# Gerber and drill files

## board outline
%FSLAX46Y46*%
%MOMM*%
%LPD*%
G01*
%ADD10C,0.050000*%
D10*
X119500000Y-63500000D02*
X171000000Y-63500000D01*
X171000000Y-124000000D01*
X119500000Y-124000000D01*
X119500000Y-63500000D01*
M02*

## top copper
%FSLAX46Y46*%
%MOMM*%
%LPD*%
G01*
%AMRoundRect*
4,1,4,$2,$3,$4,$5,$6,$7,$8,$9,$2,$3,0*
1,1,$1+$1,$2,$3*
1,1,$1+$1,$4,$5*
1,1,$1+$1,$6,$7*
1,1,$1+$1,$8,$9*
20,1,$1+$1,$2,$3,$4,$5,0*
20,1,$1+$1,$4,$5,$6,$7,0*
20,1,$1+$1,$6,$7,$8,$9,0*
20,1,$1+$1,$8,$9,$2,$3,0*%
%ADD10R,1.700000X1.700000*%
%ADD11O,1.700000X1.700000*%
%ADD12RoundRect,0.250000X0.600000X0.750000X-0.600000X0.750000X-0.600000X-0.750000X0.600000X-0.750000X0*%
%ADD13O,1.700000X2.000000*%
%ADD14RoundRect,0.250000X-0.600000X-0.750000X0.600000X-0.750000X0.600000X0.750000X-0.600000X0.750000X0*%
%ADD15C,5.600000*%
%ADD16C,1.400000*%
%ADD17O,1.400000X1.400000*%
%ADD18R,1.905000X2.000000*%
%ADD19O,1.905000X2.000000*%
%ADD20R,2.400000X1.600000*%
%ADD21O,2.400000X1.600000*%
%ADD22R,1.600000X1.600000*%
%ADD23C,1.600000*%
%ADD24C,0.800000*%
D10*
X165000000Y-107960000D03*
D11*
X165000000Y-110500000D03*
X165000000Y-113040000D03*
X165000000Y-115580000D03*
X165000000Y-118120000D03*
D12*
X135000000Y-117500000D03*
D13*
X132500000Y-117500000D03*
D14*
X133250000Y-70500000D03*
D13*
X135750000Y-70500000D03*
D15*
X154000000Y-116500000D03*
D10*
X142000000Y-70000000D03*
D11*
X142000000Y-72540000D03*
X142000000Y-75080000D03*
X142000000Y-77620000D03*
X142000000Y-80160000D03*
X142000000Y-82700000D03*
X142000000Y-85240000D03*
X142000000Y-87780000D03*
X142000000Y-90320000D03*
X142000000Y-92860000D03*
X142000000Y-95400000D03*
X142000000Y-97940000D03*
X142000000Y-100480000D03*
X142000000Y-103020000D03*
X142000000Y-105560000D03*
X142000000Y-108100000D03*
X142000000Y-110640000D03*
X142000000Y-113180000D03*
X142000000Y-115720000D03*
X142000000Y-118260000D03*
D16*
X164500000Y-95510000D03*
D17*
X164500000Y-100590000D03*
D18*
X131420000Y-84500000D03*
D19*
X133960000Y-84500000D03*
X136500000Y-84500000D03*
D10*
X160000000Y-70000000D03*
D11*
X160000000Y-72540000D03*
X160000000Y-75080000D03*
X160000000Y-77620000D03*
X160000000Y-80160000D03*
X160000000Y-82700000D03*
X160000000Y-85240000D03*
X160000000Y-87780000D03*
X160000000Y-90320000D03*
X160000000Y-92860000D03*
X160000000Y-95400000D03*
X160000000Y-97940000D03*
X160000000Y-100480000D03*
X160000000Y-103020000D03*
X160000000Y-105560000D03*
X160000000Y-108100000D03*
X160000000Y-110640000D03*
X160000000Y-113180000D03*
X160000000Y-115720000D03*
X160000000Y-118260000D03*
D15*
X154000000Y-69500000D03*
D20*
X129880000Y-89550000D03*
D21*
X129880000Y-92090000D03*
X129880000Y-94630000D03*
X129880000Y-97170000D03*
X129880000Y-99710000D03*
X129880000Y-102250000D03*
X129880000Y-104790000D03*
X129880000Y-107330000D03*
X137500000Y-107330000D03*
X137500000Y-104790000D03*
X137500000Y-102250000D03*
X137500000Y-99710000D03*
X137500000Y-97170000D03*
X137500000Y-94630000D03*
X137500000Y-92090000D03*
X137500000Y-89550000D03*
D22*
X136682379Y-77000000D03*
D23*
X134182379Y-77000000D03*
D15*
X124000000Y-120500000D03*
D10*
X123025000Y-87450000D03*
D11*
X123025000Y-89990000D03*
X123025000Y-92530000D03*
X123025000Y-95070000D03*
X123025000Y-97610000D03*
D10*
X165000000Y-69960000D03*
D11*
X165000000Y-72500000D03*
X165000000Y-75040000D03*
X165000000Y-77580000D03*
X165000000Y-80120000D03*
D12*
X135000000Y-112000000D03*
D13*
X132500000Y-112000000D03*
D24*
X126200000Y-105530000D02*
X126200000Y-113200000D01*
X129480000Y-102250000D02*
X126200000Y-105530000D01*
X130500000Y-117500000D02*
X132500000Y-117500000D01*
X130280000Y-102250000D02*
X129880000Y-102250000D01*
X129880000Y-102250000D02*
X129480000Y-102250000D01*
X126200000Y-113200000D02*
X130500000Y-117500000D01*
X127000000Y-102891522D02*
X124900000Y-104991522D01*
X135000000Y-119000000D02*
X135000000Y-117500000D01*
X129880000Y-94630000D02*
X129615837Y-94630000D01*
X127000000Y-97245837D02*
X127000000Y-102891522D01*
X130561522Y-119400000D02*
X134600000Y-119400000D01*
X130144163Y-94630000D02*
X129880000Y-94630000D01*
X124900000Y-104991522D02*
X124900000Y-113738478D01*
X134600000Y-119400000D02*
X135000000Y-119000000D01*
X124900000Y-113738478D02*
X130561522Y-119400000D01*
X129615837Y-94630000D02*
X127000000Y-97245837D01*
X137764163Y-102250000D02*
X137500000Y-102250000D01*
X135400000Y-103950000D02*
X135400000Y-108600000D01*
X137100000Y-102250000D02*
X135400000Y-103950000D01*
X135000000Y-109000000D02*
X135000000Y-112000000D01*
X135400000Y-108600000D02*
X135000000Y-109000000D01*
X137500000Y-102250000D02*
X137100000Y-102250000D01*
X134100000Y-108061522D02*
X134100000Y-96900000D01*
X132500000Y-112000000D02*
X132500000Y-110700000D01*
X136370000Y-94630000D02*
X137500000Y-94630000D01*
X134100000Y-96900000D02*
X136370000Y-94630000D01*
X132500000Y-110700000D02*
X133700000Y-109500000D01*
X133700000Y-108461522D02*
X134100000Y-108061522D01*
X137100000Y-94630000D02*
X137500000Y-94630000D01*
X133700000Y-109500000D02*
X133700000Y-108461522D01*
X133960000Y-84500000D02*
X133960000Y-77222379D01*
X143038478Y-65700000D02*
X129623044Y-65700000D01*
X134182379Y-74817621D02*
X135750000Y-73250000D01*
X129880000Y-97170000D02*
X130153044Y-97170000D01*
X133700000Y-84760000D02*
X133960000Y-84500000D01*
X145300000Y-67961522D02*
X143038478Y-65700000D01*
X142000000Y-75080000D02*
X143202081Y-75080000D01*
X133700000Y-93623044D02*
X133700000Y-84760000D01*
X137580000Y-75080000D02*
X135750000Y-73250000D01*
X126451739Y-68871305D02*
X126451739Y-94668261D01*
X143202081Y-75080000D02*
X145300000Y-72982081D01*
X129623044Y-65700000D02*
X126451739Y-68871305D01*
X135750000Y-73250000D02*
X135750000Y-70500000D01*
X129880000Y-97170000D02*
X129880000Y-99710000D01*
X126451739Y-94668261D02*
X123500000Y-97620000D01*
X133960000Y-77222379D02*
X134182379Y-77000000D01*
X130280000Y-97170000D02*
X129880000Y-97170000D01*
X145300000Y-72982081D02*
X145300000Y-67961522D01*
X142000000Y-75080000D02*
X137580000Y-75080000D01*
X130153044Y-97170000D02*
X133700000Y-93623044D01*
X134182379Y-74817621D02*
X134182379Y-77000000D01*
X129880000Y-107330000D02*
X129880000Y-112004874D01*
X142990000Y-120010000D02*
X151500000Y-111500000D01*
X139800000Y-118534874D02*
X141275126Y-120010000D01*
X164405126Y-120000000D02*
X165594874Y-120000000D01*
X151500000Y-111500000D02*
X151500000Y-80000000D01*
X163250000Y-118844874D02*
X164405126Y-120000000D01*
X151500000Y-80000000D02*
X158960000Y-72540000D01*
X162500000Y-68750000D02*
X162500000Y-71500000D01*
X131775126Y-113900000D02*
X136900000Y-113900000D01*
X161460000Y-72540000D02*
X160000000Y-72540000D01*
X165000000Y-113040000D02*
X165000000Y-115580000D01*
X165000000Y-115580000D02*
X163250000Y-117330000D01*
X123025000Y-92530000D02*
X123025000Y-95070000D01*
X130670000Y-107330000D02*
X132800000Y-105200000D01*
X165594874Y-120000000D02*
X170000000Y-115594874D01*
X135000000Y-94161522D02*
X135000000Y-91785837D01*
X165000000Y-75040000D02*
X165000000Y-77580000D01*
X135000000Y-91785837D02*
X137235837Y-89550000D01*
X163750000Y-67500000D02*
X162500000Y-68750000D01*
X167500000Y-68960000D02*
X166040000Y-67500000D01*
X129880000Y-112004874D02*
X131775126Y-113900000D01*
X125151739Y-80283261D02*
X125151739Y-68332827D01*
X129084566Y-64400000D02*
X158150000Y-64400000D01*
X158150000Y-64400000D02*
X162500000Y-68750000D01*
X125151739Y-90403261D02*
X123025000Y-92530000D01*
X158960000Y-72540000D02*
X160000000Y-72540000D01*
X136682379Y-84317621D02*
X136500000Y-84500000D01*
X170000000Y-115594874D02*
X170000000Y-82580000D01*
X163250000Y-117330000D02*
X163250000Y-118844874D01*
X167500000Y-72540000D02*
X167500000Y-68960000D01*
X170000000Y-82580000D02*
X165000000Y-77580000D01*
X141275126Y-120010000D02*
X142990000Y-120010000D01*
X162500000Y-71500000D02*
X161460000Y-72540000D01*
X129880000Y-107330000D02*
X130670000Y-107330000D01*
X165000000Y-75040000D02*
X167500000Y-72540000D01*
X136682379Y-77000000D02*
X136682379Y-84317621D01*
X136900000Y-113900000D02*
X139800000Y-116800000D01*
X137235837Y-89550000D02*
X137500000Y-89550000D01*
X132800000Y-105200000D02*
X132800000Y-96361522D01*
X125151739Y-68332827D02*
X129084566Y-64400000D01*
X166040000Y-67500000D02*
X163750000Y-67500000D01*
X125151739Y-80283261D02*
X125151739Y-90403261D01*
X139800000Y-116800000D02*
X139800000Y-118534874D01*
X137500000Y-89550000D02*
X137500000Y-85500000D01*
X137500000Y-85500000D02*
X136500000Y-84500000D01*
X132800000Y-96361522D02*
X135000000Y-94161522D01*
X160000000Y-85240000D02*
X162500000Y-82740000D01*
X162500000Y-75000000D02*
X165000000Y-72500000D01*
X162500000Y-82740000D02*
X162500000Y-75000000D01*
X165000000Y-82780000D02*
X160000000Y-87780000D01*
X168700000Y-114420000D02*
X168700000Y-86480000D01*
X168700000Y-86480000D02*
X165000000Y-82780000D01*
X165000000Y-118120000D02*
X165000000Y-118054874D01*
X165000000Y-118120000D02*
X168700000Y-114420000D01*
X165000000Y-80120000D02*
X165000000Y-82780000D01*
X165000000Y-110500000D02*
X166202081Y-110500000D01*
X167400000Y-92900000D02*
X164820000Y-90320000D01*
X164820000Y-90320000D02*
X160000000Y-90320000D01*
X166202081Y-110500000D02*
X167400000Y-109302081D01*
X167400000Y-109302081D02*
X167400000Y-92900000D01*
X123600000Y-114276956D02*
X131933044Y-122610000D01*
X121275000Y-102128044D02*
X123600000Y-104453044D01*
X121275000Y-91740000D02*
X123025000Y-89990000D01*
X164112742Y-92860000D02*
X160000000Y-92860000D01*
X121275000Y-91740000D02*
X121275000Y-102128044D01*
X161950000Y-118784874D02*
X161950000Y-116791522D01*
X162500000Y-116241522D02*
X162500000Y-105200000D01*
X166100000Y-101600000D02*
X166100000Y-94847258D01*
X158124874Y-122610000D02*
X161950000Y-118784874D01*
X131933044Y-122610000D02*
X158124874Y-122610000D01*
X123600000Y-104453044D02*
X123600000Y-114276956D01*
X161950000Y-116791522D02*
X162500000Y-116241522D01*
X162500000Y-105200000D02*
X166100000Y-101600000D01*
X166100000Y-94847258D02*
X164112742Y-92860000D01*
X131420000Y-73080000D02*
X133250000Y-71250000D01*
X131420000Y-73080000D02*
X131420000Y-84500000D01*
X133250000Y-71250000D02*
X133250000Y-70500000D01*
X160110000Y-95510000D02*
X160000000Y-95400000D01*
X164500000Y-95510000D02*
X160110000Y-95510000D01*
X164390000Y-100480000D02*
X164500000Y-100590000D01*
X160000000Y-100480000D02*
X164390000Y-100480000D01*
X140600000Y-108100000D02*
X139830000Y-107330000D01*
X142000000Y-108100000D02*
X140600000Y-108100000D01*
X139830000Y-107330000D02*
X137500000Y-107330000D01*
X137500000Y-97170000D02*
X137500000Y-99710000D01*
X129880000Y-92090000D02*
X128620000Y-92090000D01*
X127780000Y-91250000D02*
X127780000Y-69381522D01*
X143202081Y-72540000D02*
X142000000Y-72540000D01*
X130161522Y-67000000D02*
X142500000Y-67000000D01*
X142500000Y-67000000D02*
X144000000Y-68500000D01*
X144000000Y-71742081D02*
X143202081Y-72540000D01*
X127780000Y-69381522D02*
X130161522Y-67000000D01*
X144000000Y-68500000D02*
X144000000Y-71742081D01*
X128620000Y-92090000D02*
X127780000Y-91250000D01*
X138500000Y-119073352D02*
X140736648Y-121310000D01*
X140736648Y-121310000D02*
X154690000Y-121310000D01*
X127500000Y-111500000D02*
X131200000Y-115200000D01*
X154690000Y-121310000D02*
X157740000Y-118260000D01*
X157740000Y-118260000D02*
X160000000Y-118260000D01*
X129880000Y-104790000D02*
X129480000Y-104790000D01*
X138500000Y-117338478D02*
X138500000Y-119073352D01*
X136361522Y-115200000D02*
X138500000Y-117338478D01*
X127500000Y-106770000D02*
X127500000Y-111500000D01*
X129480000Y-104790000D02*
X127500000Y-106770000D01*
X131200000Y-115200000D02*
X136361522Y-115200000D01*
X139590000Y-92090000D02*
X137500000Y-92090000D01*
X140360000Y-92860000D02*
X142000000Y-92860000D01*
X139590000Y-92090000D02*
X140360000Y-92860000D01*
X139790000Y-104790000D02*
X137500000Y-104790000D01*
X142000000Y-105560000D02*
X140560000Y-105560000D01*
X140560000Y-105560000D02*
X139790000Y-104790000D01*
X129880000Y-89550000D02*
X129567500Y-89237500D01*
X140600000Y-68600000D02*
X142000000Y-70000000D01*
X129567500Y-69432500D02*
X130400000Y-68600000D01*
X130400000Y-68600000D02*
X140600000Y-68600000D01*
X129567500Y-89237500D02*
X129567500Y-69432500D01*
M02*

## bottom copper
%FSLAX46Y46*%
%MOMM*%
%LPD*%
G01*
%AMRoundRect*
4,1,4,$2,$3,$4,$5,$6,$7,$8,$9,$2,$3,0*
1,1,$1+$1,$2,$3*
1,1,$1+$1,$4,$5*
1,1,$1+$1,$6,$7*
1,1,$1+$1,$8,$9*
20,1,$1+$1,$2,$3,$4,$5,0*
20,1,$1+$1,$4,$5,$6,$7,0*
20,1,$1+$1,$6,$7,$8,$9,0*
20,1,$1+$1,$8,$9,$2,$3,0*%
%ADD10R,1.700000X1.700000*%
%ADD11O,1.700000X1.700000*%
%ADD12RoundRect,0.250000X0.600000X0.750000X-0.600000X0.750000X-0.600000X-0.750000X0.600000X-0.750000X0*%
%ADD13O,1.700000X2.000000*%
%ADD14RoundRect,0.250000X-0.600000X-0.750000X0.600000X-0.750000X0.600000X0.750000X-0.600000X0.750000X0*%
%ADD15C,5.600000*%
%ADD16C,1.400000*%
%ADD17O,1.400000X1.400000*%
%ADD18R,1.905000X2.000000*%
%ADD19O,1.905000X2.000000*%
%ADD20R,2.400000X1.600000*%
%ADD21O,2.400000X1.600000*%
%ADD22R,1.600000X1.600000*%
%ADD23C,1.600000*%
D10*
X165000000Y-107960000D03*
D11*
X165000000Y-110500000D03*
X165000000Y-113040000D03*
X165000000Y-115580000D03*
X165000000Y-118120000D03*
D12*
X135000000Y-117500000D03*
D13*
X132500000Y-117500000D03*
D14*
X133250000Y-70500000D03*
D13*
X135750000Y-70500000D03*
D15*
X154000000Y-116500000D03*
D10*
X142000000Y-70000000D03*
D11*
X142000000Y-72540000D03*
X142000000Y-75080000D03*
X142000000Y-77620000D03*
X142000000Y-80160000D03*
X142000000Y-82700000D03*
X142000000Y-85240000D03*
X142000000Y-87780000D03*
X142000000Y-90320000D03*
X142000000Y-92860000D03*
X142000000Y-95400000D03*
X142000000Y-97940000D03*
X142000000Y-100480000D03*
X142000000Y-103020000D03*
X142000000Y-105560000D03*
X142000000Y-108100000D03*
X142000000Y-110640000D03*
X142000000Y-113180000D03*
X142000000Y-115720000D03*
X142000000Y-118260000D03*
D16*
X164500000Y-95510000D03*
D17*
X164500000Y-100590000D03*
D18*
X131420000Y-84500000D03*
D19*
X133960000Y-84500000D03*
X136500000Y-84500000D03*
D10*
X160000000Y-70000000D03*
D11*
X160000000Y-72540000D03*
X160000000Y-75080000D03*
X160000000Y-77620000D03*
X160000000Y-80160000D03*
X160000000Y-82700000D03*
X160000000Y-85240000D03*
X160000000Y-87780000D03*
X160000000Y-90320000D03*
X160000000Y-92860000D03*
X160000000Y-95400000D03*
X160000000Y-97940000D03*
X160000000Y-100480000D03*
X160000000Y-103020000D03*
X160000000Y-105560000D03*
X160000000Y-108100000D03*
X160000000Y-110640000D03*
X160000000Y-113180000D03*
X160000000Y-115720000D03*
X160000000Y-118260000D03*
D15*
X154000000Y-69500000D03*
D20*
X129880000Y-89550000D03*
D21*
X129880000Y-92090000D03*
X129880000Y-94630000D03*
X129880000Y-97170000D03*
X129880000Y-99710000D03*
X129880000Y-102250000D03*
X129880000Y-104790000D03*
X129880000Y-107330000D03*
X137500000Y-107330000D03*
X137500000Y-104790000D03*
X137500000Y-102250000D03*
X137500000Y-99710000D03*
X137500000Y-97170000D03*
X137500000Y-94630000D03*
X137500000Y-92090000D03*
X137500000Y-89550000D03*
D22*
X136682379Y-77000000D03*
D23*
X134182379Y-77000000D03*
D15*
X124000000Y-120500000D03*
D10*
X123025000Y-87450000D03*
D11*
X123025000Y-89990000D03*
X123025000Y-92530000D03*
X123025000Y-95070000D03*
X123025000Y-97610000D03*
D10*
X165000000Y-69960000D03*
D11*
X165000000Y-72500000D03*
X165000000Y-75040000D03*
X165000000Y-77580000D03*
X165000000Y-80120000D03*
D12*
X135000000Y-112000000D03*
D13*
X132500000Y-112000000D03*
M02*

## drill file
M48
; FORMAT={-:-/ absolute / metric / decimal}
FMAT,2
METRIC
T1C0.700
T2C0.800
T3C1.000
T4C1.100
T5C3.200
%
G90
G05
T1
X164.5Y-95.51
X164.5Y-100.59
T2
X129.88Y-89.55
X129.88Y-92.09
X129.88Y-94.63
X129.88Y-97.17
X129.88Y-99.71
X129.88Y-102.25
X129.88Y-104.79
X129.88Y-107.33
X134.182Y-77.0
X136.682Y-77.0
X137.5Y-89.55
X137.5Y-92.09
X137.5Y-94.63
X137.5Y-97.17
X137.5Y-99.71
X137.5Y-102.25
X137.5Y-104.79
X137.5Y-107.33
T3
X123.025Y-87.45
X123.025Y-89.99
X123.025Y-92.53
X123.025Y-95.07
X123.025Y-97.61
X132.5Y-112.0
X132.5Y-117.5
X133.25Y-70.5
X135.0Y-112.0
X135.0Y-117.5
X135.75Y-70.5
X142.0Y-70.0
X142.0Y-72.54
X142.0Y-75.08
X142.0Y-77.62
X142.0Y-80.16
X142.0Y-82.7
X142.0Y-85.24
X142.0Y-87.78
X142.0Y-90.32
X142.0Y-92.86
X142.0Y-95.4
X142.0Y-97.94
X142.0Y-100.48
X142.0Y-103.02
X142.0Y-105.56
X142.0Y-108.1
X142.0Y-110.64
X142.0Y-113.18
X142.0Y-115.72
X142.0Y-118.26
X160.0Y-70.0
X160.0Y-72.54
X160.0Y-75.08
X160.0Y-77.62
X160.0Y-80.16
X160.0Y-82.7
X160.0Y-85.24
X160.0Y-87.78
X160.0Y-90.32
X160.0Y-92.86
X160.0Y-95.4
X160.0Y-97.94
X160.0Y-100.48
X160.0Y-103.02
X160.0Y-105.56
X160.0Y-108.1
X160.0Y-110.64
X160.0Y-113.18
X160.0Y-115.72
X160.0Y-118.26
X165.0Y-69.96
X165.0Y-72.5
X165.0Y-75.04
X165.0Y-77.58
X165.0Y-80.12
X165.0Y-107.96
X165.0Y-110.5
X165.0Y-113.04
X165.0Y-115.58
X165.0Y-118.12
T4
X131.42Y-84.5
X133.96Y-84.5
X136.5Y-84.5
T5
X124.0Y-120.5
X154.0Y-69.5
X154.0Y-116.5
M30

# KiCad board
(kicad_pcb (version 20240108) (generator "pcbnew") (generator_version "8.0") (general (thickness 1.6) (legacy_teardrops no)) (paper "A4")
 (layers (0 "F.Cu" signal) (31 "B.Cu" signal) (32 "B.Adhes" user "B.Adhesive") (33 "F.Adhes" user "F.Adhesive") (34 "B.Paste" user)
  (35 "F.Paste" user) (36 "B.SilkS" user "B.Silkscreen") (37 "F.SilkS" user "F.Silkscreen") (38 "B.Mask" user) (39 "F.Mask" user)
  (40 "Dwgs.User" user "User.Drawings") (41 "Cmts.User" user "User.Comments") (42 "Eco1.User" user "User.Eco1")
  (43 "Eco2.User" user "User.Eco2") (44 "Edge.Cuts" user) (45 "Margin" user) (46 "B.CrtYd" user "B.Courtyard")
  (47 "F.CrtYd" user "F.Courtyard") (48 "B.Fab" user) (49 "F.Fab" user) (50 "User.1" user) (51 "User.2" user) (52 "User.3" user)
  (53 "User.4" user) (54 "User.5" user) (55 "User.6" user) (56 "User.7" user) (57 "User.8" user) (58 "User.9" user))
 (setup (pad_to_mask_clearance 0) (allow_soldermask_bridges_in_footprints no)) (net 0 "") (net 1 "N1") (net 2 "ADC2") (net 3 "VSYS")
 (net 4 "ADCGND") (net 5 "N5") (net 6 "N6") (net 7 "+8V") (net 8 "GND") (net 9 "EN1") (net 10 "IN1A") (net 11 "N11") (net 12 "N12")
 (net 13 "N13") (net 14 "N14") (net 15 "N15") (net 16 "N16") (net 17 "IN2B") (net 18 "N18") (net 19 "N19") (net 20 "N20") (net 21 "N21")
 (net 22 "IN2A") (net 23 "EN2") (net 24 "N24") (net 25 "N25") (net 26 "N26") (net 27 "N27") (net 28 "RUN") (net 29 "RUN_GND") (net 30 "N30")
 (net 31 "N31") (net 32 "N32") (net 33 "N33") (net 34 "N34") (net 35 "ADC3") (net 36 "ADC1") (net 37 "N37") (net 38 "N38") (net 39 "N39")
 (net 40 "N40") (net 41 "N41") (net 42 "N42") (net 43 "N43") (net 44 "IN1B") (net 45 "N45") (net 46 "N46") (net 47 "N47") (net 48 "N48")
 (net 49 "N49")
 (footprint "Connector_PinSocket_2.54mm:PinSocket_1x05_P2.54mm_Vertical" (layer "F.Cu") (at 165 107.96)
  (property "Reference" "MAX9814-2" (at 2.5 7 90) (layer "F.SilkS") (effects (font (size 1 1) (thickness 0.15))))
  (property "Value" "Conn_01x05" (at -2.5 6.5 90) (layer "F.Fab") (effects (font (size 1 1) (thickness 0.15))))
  (pad "1" thru_hole rect (at 0 0) (size 1.7 1.7) (drill 1) (layers "*.Cu" "*.Mask") (remove_unused_layers no) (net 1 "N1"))
  (pad "2" thru_hole oval (at 0 2.54) (size 1.7 1.7) (drill 1) (layers "*.Cu" "*.Mask") (remove_unused_layers no) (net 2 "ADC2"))
  (pad "3" thru_hole oval (at 0 5.08) (size 1.7 1.7) (drill 1) (layers "*.Cu" "*.Mask") (remove_unused_layers no) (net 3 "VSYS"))
  (pad "4" thru_hole oval (at 0 7.62) (size 1.7 1.7) (drill 1) (layers "*.Cu" "*.Mask") (remove_unused_layers no) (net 3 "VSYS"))
  (pad "5" thru_hole oval (at 0 10.16) (size 1.7 1.7) (drill 1) (layers "*.Cu" "*.Mask") (remove_unused_layers no) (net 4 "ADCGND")))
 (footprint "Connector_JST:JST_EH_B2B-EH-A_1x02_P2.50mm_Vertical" (layer "F.Cu") (at 135 117.5 180)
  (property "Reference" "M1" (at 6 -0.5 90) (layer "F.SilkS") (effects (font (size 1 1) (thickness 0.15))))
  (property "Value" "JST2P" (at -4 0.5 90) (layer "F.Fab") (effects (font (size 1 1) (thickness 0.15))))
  (pad "1" thru_hole roundrect (at 0 0 180) (size 1.7 2) (drill 1) (layers "*.Cu" "*.Mask") (remove_unused_layers no)
   (roundrect_rratio 0.147059) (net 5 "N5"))
  (pad "2" thru_hole oval (at 2.5 0 180) (size 1.7 2) (drill 1) (layers "*.Cu" "*.Mask") (remove_unused_layers no) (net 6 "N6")))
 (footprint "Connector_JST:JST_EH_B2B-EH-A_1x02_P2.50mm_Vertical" (layer "F.Cu") (at 133.25 70.5)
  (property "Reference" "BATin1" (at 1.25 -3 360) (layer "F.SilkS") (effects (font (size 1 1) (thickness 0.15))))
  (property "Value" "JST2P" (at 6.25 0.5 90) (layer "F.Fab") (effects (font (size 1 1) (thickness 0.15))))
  (pad "1" thru_hole roundrect (at 0 0) (size 1.7 2) (drill 1) (layers "*.Cu" "*.Mask") (remove_unused_layers no)
   (roundrect_rratio 0.147059) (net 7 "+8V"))
  (pad "2" thru_hole oval (at 2.5 0) (size 1.7 2) (drill 1) (layers "*.Cu" "*.Mask") (remove_unused_layers no) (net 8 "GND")))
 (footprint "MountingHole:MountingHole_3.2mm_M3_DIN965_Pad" (layer "F.Cu") (at 154 116.5)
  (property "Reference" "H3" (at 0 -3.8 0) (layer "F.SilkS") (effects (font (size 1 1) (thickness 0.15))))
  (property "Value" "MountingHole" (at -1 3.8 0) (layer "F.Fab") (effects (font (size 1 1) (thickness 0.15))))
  (pad "1" thru_hole circle (at 0 0) (size 5.6 5.6) (drill 3.2) (layers "*.Cu" "*.Mask") (remove_unused_layers no)))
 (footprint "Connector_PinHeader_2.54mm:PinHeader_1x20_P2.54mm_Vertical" (layer "F.Cu") (at 142 70)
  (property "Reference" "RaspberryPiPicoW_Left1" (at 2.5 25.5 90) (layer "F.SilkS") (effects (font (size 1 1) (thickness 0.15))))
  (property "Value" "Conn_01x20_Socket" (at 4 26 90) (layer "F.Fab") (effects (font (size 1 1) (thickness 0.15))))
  (pad "1" thru_hole rect (at 0 0) (size 1.7 1.7) (drill 1) (layers "*.Cu" "*.Mask") (remove_unused_layers no) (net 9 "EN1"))
  (pad "2" thru_hole oval (at 0 2.54) (size 1.7 1.7) (drill 1) (layers "*.Cu" "*.Mask") (remove_unused_layers no) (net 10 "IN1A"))
  (pad "3" thru_hole oval (at 0 5.08) (size 1.7 1.7) (drill 1) (layers "*.Cu" "*.Mask") (remove_unused_layers no) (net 8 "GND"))
  (pad "4" thru_hole oval (at 0 7.62) (size 1.7 1.7) (drill 1) (layers "*.Cu" "*.Mask") (remove_unused_layers no) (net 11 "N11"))
  (pad "5" thru_hole oval (at 0 10.16) (size 1.7 1.7) (drill 1) (layers "*.Cu" "*.Mask") (remove_unused_layers no) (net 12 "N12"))
  (pad "6" thru_hole oval (at 0 12.7) (size 1.7 1.7) (drill 1) (layers "*.Cu" "*.Mask") (remove_unused_layers no) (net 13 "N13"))
  (pad "7" thru_hole oval (at 0 15.24) (size 1.7 1.7) (drill 1) (layers "*.Cu" "*.Mask") (remove_unused_layers no) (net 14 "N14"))
  (pad "8" thru_hole oval (at 0 17.78) (size 1.7 1.7) (drill 1) (layers "*.Cu" "*.Mask") (remove_unused_layers no) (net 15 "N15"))
  (pad "9" thru_hole oval (at 0 20.32) (size 1.7 1.7) (drill 1) (layers "*.Cu" "*.Mask") (remove_unused_layers no) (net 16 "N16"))
  (pad "10" thru_hole oval (at 0 22.86) (size 1.7 1.7) (drill 1) (layers "*.Cu" "*.Mask") (remove_unused_layers no) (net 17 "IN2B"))
  (pad "11" thru_hole oval (at 0 25.4) (size 1.7 1.7) (drill 1) (layers "*.Cu" "*.Mask") (remove_unused_layers no) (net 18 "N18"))
  (pad "12" thru_hole oval (at 0 27.94) (size 1.7 1.7) (drill 1) (layers "*.Cu" "*.Mask") (remove_unused_layers no) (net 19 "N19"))
  (pad "13" thru_hole oval (at 0 30.48) (size 1.7 1.7) (drill 1) (layers "*.Cu" "*.Mask") (remove_unused_layers no) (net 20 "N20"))
  (pad "14" thru_hole oval (at 0 33.02) (size 1.7 1.7) (drill 1) (layers "*.Cu" "*.Mask") (remove_unused_layers no) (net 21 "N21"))
  (pad "15" thru_hole oval (at 0 35.56) (size 1.7 1.7) (drill 1) (layers "*.Cu" "*.Mask") (remove_unused_layers no) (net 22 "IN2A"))
  (pad "16" thru_hole oval (at 0 38.1) (size 1.7 1.7) (drill 1) (layers "*.Cu" "*.Mask") (remove_unused_layers no) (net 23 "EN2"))
  (pad "17" thru_hole oval (at 0 40.64) (size 1.7 1.7) (drill 1) (layers "*.Cu" "*.Mask") (remove_unused_layers no) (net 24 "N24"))
  (pad "18" thru_hole oval (at 0 43.18) (size 1.7 1.7) (drill 1) (layers "*.Cu" "*.Mask") (remove_unused_layers no) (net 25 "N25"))
  (pad "19" thru_hole oval (at 0 45.72) (size 1.7 1.7) (drill 1) (layers "*.Cu" "*.Mask") (remove_unused_layers no) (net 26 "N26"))
  (pad "20" thru_hole oval (at 0 48.26) (size 1.7 1.7) (drill 1) (layers "*.Cu" "*.Mask") (remove_unused_layers no) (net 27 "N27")))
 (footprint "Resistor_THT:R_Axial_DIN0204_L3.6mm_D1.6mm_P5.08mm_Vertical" (layer "F.Cu") (at 164.5 95.51 -90)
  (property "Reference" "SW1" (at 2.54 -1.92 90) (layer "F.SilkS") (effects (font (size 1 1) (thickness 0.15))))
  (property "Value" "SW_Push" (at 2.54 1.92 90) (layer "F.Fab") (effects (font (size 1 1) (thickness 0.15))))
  (pad "1" thru_hole circle (at 0 0 270) (size 1.4 1.4) (drill 0.7) (layers "*.Cu" "*.Mask") (remove_unused_layers no) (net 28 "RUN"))
  (pad "2" thru_hole oval (at 5.08 0 270) (size 1.4 1.4) (drill 0.7) (layers "*.Cu" "*.Mask") (remove_unused_layers no) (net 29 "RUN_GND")))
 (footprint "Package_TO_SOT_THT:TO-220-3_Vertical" (layer "F.Cu") (at 131.42 84.5)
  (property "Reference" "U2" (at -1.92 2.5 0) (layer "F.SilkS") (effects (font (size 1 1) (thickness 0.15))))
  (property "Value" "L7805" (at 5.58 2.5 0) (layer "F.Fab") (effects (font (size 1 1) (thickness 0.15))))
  (pad "1" thru_hole rect (at 0 0) (size 1.905 2) (drill 1.1) (layers "*.Cu" "*.Mask") (remove_unused_layers no) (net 7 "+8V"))
  (pad "2" thru_hole oval (at 2.54 0) (size 1.905 2) (drill 1.1) (layers "*.Cu" "*.Mask") (remove_unused_layers no) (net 8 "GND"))
  (pad "3" thru_hole oval (at 5.08 0) (size 1.905 2) (drill 1.1) (layers "*.Cu" "*.Mask") (remove_unused_layers no) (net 3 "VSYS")))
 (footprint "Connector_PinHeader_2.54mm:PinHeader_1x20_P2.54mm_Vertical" (layer "F.Cu") (at 160 70)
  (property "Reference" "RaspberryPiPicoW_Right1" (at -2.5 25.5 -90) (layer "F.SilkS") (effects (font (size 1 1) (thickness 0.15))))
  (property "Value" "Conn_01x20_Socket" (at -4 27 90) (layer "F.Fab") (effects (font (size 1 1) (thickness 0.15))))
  (pad "1" thru_hole rect (at 0 0) (size 1.7 1.7) (drill 1) (layers "*.Cu" "*.Mask") (remove_unused_layers no) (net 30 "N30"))
  (pad "2" thru_hole oval (at 0 2.54) (size 1.7 1.7) (drill 1) (layers "*.Cu" "*.Mask") (remove_unused_layers no) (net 3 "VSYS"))
  (pad "3" thru_hole oval (at 0 5.08) (size 1.7 1.7) (drill 1) (layers "*.Cu" "*.Mask") (remove_unused_layers no) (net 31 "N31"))
  (pad "4" thru_hole oval (at 0 7.62) (size 1.7 1.7) (drill 1) (layers "*.Cu" "*.Mask") (remove_unused_layers no) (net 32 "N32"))
  (pad "5" thru_hole oval (at 0 10.16) (size 1.7 1.7) (drill 1) (layers "*.Cu" "*.Mask") (remove_unused_layers no) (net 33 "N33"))
  (pad "6" thru_hole oval (at 0 12.7) (size 1.7 1.7) (drill 1) (layers "*.Cu" "*.Mask") (remove_unused_layers no) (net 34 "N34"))
  (pad "7" thru_hole oval (at 0 15.24) (size 1.7 1.7) (drill 1) (layers "*.Cu" "*.Mask") (remove_unused_layers no) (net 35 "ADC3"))
  (pad "8" thru_hole oval (at 0 17.78) (size 1.7 1.7) (drill 1) (layers "*.Cu" "*.Mask") (remove_unused_layers no) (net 4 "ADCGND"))
  (pad "9" thru_hole oval (at 0 20.32) (size 1.7 1.7) (drill 1) (layers "*.Cu" "*.Mask") (remove_unused_layers no) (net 2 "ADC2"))
  (pad "10" thru_hole oval (at 0 22.86) (size 1.7 1.7) (drill 1) (layers "*.Cu" "*.Mask") (remove_unused_layers no) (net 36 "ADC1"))
  (pad "11" thru_hole oval (at 0 25.4) (size 1.7 1.7) (drill 1) (layers "*.Cu" "*.Mask") (remove_unused_layers no) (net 28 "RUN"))
  (pad "12" thru_hole oval (at 0 27.94) (size 1.7 1.7) (drill 1) (layers "*.Cu" "*.Mask") (remove_unused_layers no) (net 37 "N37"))
  (pad "13" thru_hole oval (at 0 30.48) (size 1.7 1.7) (drill 1) (layers "*.Cu" "*.Mask") (remove_unused_layers no) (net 29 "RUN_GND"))
  (pad "14" thru_hole oval (at 0 33.02) (size 1.7 1.7) (drill 1) (layers "*.Cu" "*.Mask") (remove_unused_layers no) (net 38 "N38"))
  (pad "15" thru_hole oval (at 0 35.56) (size 1.7 1.7) (drill 1) (layers "*.Cu" "*.Mask") (remove_unused_layers no) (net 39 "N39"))
  (pad "16" thru_hole oval (at 0 38.1) (size 1.7 1.7) (drill 1) (layers "*.Cu" "*.Mask") (remove_unused_layers no) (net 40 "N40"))
  (pad "17" thru_hole oval (at 0 40.64) (size 1.7 1.7) (drill 1) (layers "*.Cu" "*.Mask") (remove_unused_layers no) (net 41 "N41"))
  (pad "18" thru_hole oval (at 0 43.18) (size 1.7 1.7) (drill 1) (layers "*.Cu" "*.Mask") (remove_unused_layers no) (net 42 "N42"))
  (pad "19" thru_hole oval (at 0 45.72) (size 1.7 1.7) (drill 1) (layers "*.Cu" "*.Mask") (remove_unused_layers no) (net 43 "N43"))
  (pad "20" thru_hole oval (at 0 48.26) (size 1.7 1.7) (drill 1) (layers "*.Cu" "*.Mask") (remove_unused_layers no) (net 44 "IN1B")))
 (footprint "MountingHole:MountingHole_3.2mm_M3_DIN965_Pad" (layer "F.Cu") (at 154 69.5)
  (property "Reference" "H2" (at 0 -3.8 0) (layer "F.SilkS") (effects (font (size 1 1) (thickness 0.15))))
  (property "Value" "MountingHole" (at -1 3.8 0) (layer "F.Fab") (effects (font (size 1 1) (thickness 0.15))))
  (pad "1" thru_hole circle (at 0 0) (size 5.6 5.6) (drill 3.2) (layers "*.Cu" "*.Mask") (remove_unused_layers no)))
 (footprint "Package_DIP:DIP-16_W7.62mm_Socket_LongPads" (layer "F.Cu") (at 129.88 89.55)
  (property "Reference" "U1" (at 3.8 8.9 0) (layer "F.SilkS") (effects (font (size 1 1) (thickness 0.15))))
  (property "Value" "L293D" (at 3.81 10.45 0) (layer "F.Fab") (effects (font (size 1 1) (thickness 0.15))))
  (pad "1" thru_hole rect (at 0 0) (size 2.4 1.6) (drill 0.8) (layers "*.Cu" "*.Mask") (remove_unused_layers no) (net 9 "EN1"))
  (pad "2" thru_hole oval (at 0 2.54) (size 2.4 1.6) (drill 0.8) (layers "*.Cu" "*.Mask") (remove_unused_layers no) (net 10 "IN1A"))
  (pad "3" thru_hole oval (at 0 5.08) (size 2.4 1.6) (drill 0.8) (layers "*.Cu" "*.Mask") (remove_unused_layers no) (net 5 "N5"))
  (pad "4" thru_hole oval (at 0 7.62) (size 2.4 1.6) (drill 0.8) (layers "*.Cu" "*.Mask") (remove_unused_layers no) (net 8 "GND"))
  (pad "5" thru_hole oval (at 0 10.16) (size 2.4 1.6) (drill 0.8) (layers "*.Cu" "*.Mask") (remove_unused_layers no) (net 8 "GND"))
  (pad "6" thru_hole oval (at 0 12.7) (size 2.4 1.6) (drill 0.8) (layers "*.Cu" "*.Mask") (remove_unused_layers no) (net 6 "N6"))
  (pad "7" thru_hole oval (at 0 15.24) (size 2.4 1.6) (drill 0.8) (layers "*.Cu" "*.Mask") (remove_unused_layers no) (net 44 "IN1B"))
  (pad "8" thru_hole oval (at 0 17.78) (size 2.4 1.6) (drill 0.8) (layers "*.Cu" "*.Mask") (remove_unused_layers no) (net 3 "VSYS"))
  (pad "9" thru_hole oval (at 7.62 17.78) (size 2.4 1.6) (drill 0.8) (layers "*.Cu" "*.Mask") (remove_unused_layers no) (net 23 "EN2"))
  (pad "10" thru_hole oval (at 7.62 15.24) (size 2.4 1.6) (drill 0.8) (layers "*.Cu" "*.Mask") (remove_unused_layers no) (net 22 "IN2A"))
  (pad "11" thru_hole oval (at 7.62 12.7) (size 2.4 1.6) (drill 0.8) (layers "*.Cu" "*.Mask") (remove_unused_layers no) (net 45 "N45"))
  (pad "12" thru_hole oval (at 7.62 10.16) (size 2.4 1.6) (drill 0.8) (layers "*.Cu" "*.Mask") (remove_unused_layers no) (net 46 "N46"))
  (pad "13" thru_hole oval (at 7.62 7.62) (size 2.4 1.6) (drill 0.8) (layers "*.Cu" "*.Mask") (remove_unused_layers no) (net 46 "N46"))
  (pad "14" thru_hole oval (at 7.62 5.08) (size 2.4 1.6) (drill 0.8) (layers "*.Cu" "*.Mask") (remove_unused_layers no) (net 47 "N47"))
  (pad "15" thru_hole oval (at 7.62 2.54) (size 2.4 1.6) (drill 0.8) (layers "*.Cu" "*.Mask") (remove_unused_layers no) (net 17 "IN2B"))
  (pad "16" thru_hole oval (at 7.62 0) (size 2.4 1.6) (drill 0.8) (layers "*.Cu" "*.Mask") (remove_unused_layers no) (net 3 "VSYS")))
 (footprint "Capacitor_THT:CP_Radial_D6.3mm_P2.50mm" (layer "F.Cu") (at 136.682379 77 180)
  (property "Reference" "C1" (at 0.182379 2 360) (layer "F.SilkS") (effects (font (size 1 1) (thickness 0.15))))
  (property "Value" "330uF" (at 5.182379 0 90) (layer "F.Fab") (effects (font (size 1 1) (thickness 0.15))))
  (pad "1" thru_hole rect (at 0 0 180) (size 1.6 1.6) (drill 0.8) (layers "*.Cu" "*.Mask") (remove_unused_layers no) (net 3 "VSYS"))
  (pad "2" thru_hole circle (at 2.5 0 180) (size 1.6 1.6) (drill 0.8) (layers "*.Cu" "*.Mask") (remove_unused_layers no) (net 8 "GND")))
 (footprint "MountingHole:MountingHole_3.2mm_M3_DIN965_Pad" (layer "F.Cu") (at 124 120.5)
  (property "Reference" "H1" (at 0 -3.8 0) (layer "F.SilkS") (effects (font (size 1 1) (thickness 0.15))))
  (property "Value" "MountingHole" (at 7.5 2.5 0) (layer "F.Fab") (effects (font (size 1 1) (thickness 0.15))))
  (pad "1" thru_hole circle (at 0 0) (size 5.6 5.6) (drill 3.2) (layers "*.Cu" "*.Mask") (remove_unused_layers no)))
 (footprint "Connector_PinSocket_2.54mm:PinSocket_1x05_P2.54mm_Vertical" (layer "F.Cu") (at 123.025 87.45)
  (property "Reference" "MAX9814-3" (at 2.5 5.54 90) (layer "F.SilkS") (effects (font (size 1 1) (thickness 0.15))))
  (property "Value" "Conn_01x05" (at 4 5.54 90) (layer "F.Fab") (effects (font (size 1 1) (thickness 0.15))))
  (pad "1" thru_hole rect (at 0 0) (size 1.7 1.7) (drill 1) (layers "*.Cu" "*.Mask") (remove_unused_layers no) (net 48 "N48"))
  (pad "2" thru_hole oval (at 0 2.54) (size 1.7 1.7) (drill 1) (layers "*.Cu" "*.Mask") (remove_unused_layers no) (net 36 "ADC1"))
  (pad "3" thru_hole oval (at 0 5.08) (size 1.7 1.7) (drill 1) (layers "*.Cu" "*.Mask") (remove_unused_layers no) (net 3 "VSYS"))
  (pad "4" thru_hole oval (at 0 7.62) (size 1.7 1.7) (drill 1) (layers "*.Cu" "*.Mask") (remove_unused_layers no) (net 3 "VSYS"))
  (pad "5" thru_hole oval (at 0 10.16) (size 1.7 1.7) (drill 1) (layers "*.Cu" "*.Mask") (remove_unused_layers no) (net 8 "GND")))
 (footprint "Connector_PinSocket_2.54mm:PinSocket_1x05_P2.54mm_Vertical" (layer "F.Cu") (at 165 69.96)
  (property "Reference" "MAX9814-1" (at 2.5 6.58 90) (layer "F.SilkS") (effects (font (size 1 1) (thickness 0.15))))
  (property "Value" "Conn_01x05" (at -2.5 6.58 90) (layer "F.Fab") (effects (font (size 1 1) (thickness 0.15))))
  (pad "1" thru_hole rect (at 0 0) (size 1.7 1.7) (drill 1) (layers "*.Cu" "*.Mask") (remove_unused_layers no) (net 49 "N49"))
  (pad "2" thru_hole oval (at 0 2.54) (size 1.7 1.7) (drill 1) (layers "*.Cu" "*.Mask") (remove_unused_layers no) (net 35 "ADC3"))
  (pad "3" thru_hole oval (at 0 5.08) (size 1.7 1.7) (drill 1) (layers "*.Cu" "*.Mask") (remove_unused_layers no) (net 3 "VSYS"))
  (pad "4" thru_hole oval (at 0 7.62) (size 1.7 1.7) (drill 1) (layers "*.Cu" "*.Mask") (remove_unused_layers no) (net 3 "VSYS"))
  (pad "5" thru_hole oval (at 0 10.16) (size 1.7 1.7) (drill 1) (layers "*.Cu" "*.Mask") (remove_unused_layers no) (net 4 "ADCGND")))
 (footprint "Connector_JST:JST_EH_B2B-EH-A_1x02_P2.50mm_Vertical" (layer "F.Cu") (at 135 112 180)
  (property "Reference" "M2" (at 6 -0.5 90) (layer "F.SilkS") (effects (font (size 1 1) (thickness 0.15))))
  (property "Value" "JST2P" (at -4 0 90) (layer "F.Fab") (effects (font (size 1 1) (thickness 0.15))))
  (pad "1" thru_hole roundrect (at 0 0 180) (size 1.7 2) (drill 1) (layers "*.Cu" "*.Mask") (remove_unused_layers no)
   (roundrect_rratio 0.147059) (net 45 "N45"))
  (pad "2" thru_hole oval (at 2.5 0 180) (size 1.7 2) (drill 1) (layers "*.Cu" "*.Mask") (remove_unused_layers no) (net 47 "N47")))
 (gr_rect (start 119.5 63.5) (end 171 124) (stroke (width 0.05) (type default)) (fill none) (layer "Edge.Cuts"))
 (segment (start 126.2 105.53) (end 126.2 113.2) (width 0.8) (layer "F.Cu") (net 6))
 (segment (start 129.48 102.25) (end 126.2 105.53) (width 0.8) (layer "F.Cu") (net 6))
 (segment (start 130.5 117.5) (end 132.5 117.5) (width 0.8) (layer "F.Cu") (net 6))
 (segment (start 130.28 102.25) (end 129.88 102.25) (width 0.8) (layer "F.Cu") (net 6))
 (segment (start 129.88 102.25) (end 129.48 102.25) (width 0.8) (layer "F.Cu") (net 6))
 (segment (start 126.2 113.2) (end 130.5 117.5) (width 0.8) (layer "F.Cu") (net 6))
 (segment (start 127 102.891522) (end 124.9 104.991522) (width 0.8) (layer "F.Cu") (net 5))
 (segment (start 135 119) (end 135 117.5) (width 0.8) (layer "F.Cu") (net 5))
 (segment (start 129.88 94.63) (end 129.615837 94.63) (width 0.8) (layer "F.Cu") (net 5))
 (segment (start 127 97.245837) (end 127 102.891522) (width 0.8) (layer "F.Cu") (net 5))
 (segment (start 130.561522 119.4) (end 134.6 119.4) (width 0.8) (layer "F.Cu") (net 5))
 (segment (start 130.144163 94.63) (end 129.88 94.63) (width 0.8) (layer "F.Cu") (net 5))
 (segment (start 124.9 104.991522) (end 124.9 113.738478) (width 0.8) (layer "F.Cu") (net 5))
 (segment (start 134.6 119.4) (end 135 119) (width 0.8) (layer "F.Cu") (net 5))
 (segment (start 124.9 113.738478) (end 130.561522 119.4) (width 0.8) (layer "F.Cu") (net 5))
 (segment (start 129.615837 94.63) (end 127 97.245837) (width 0.8) (layer "F.Cu") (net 5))
 (segment (start 137.764163 102.25) (end 137.5 102.25) (width 0.8) (layer "F.Cu") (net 45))
 (segment (start 135.4 103.95) (end 135.4 108.6) (width 0.8) (layer "F.Cu") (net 45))
 (segment (start 137.1 102.25) (end 135.4 103.95) (width 0.8) (layer "F.Cu") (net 45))
 (segment (start 135 109) (end 135 112) (width 0.8) (layer "F.Cu") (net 45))
 (segment (start 135.4 108.6) (end 135 109) (width 0.8) (layer "F.Cu") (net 45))
 (segment (start 137.5 102.25) (end 137.1 102.25) (width 0.8) (layer "F.Cu") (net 45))
 (segment (start 134.1 108.061522) (end 134.1 96.9) (width 0.8) (layer "F.Cu") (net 47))
 (segment (start 132.5 112) (end 132.5 110.7) (width 0.8) (layer "F.Cu") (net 47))
 (segment (start 136.37 94.63) (end 137.5 94.63) (width 0.8) (layer "F.Cu") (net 47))
 (segment (start 134.1 96.9) (end 136.37 94.63) (width 0.8) (layer "F.Cu") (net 47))
 (segment (start 132.5 110.7) (end 133.7 109.5) (width 0.8) (layer "F.Cu") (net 47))
 (segment (start 133.7 108.461522) (end 134.1 108.061522) (width 0.8) (layer "F.Cu") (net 47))
 (segment (start 137.1 94.63) (end 137.5 94.63) (width 0.8) (layer "F.Cu") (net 47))
 (segment (start 133.7 109.5) (end 133.7 108.461522) (width 0.8) (layer "F.Cu") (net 47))
 (segment (start 133.96 84.5) (end 133.96 77.222379) (width 0.8) (layer "F.Cu") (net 8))
 (segment (start 143.038478 65.7) (end 129.623044 65.7) (width 0.8) (layer "F.Cu") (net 8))
 (segment (start 134.182379 74.817621) (end 135.75 73.25) (width 0.8) (layer "F.Cu") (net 8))
 (segment (start 129.88 97.17) (end 130.153044 97.17) (width 0.8) (layer "F.Cu") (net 8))
 (segment (start 133.7 84.76) (end 133.96 84.5) (width 0.8) (layer "F.Cu") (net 8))
 (segment (start 145.3 67.961522) (end 143.038478 65.7) (width 0.8) (layer "F.Cu") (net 8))
 (segment (start 142 75.08) (end 143.202081 75.08) (width 0.8) (layer "F.Cu") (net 8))
 (segment (start 133.7 93.623044) (end 133.7 84.76) (width 0.8) (layer "F.Cu") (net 8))
 (segment (start 137.58 75.08) (end 135.75 73.25) (width 0.8) (layer "F.Cu") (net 8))
 (segment (start 126.451739 68.871305) (end 126.451739 94.668261) (width 0.8) (layer "F.Cu") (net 8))
 (segment (start 143.202081 75.08) (end 145.3 72.982081) (width 0.8) (layer "F.Cu") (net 8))
 (segment (start 129.623044 65.7) (end 126.451739 68.871305) (width 0.8) (layer "F.Cu") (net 8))
 (segment (start 135.75 73.25) (end 135.75 70.5) (width 0.8) (layer "F.Cu") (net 8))
 (segment (start 129.88 97.17) (end 129.88 99.71) (width 0.8) (layer "F.Cu") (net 8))
 (segment (start 126.451739 94.668261) (end 123.5 97.62) (width 0.8) (layer "F.Cu") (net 8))
 (segment (start 133.96 77.222379) (end 134.182379 77) (width 0.8) (layer "F.Cu") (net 8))
 (segment (start 130.28 97.17) (end 129.88 97.17) (width 0.8) (layer "F.Cu") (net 8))
 (segment (start 145.3 72.982081) (end 145.3 67.961522) (width 0.8) (layer "F.Cu") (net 8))
 (segment (start 142 75.08) (end 137.58 75.08) (width 0.8) (layer "F.Cu") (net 8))
 (segment (start 130.153044 97.17) (end 133.7 93.623044) (width 0.8) (layer "F.Cu") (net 8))
 (segment (start 134.182379 74.817621) (end 134.182379 77) (width 0.8) (layer "F.Cu") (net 8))
 (segment (start 129.88 107.33) (end 129.88 112.004874) (width 0.8) (layer "F.Cu") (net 3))
 (segment (start 142.99 120.01) (end 151.5 111.5) (width 0.8) (layer "F.Cu") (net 3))
 (segment (start 139.8 118.534874) (end 141.275126 120.01) (width 0.8) (layer "F.Cu") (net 3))
 (segment (start 164.405126 120) (end 165.594874 120) (width 0.8) (layer "F.Cu") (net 3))
 (segment (start 151.5 111.5) (end 151.5 80) (width 0.8) (layer "F.Cu") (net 3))
 (segment (start 163.25 118.844874) (end 164.405126 120) (width 0.8) (layer "F.Cu") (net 3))
 (segment (start 151.5 80) (end 158.96 72.54) (width 0.8) (layer "F.Cu") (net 3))
 (segment (start 162.5 68.75) (end 162.5 71.5) (width 0.8) (layer "F.Cu") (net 3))
 (segment (start 131.775126 113.9) (end 136.9 113.9) (width 0.8) (layer "F.Cu") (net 3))
 (segment (start 161.46 72.54) (end 160 72.54) (width 0.8) (layer "F.Cu") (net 3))
 (segment (start 165 113.04) (end 165 115.58) (width 0.8) (layer "F.Cu") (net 3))
 (segment (start 165 115.58) (end 163.25 117.33) (width 0.8) (layer "F.Cu") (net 3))
 (segment (start 123.025 92.53) (end 123.025 95.07) (width 0.8) (layer "F.Cu") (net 3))
 (segment (start 130.67 107.33) (end 132.8 105.2) (width 0.8) (layer "F.Cu") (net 3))
 (segment (start 165.594874 120) (end 170 115.594874) (width 0.8) (layer "F.Cu") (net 3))
 (segment (start 135 94.161522) (end 135 91.785837) (width 0.8) (layer "F.Cu") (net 3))
 (segment (start 165 75.04) (end 165 77.58) (width 0.8) (layer "F.Cu") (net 3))
 (segment (start 135 91.785837) (end 137.235837 89.55) (width 0.8) (layer "F.Cu") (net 3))
 (segment (start 163.75 67.5) (end 162.5 68.75) (width 0.8) (layer "F.Cu") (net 3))
 (segment (start 167.5 68.96) (end 166.04 67.5) (width 0.8) (layer "F.Cu") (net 3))
 (segment (start 129.88 112.004874) (end 131.775126 113.9) (width 0.8) (layer "F.Cu") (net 3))
 (segment (start 125.151739 80.283261) (end 125.151739 68.332827) (width 0.8) (layer "F.Cu") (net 3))
 (segment (start 129.084566 64.4) (end 158.15 64.4) (width 0.8) (layer "F.Cu") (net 3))
 (segment (start 158.15 64.4) (end 162.5 68.75) (width 0.8) (layer "F.Cu") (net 3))
 (segment (start 125.151739 90.403261) (end 123.025 92.53) (width 0.8) (layer "F.Cu") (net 3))
 (segment (start 158.96 72.54) (end 160 72.54) (width 0.8) (layer "F.Cu") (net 3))
 (segment (start 136.682379 84.317621) (end 136.5 84.5) (width 0.8) (layer "F.Cu") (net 3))
 (segment (start 170 115.594874) (end 170 82.58) (width 0.8) (layer "F.Cu") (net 3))
 (segment (start 163.25 117.33) (end 163.25 118.844874) (width 0.8) (layer "F.Cu") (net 3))
 (segment (start 167.5 72.54) (end 167.5 68.96) (width 0.8) (layer "F.Cu") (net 3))
 (segment (start 170 82.58) (end 165 77.58) (width 0.8) (layer "F.Cu") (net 3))
 (segment (start 141.275126 120.01) (end 142.99 120.01) (width 0.8) (layer "F.Cu") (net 3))
 (segment (start 162.5 71.5) (end 161.46 72.54) (width 0.8) (layer "F.Cu") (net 3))
 (segment (start 129.88 107.33) (end 130.67 107.33) (width 0.8) (layer "F.Cu") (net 3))
 (segment (start 165 75.04) (end 167.5 72.54) (width 0.8) (layer "F.Cu") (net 3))
 (segment (start 136.682379 77) (end 136.682379 84.317621) (width 0.8) (layer "F.Cu") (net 3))
 (segment (start 136.9 113.9) (end 139.8 116.8) (width 0.8) (layer "F.Cu") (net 3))
 (segment (start 137.235837 89.55) (end 137.5 89.55) (width 0.8) (layer "F.Cu") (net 3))
 (segment (start 132.8 105.2) (end 132.8 96.361522) (width 0.8) (layer "F.Cu") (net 3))
 (segment (start 125.151739 68.332827) (end 129.084566 64.4) (width 0.8) (layer "F.Cu") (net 3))
 (segment (start 166.04 67.5) (end 163.75 67.5) (width 0.8) (layer "F.Cu") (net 3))
 (segment (start 125.151739 80.283261) (end 125.151739 90.403261) (width 0.8) (layer "F.Cu") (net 3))
 (segment (start 139.8 116.8) (end 139.8 118.534874) (width 0.8) (layer "F.Cu") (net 3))
 (segment (start 137.5 89.55) (end 137.5 85.5) (width 0.8) (layer "F.Cu") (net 3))
 (segment (start 137.5 85.5) (end 136.5 84.5) (width 0.8) (layer "F.Cu") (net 3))
 (segment (start 132.8 96.361522) (end 135 94.161522) (width 0.8) (layer "F.Cu") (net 3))
 (segment (start 160 85.24) (end 162.5 82.74) (width 0.8) (layer "F.Cu") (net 35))
 (segment (start 162.5 75) (end 165 72.5) (width 0.8) (layer "F.Cu") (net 35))
 (segment (start 162.5 82.74) (end 162.5 75) (width 0.8) (layer "F.Cu") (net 35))
 (segment (start 165 82.78) (end 160 87.78) (width 0.8) (layer "F.Cu") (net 4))
 (segment (start 168.7 114.42) (end 168.7 86.48) (width 0.8) (layer "F.Cu") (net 4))
 (segment (start 168.7 86.48) (end 165 82.78) (width 0.8) (layer "F.Cu") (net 4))
 (segment (start 165 118.12) (end 165 118.054874) (width 0.8) (layer "F.Cu") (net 4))
 (segment (start 165 118.12) (end 168.7 114.42) (width 0.8) (layer "F.Cu") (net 4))
 (segment (start 165 80.12) (end 165 82.78) (width 0.8) (layer "F.Cu") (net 4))
 (segment (start 165 110.5) (end 166.202081 110.5) (width 0.8) (layer "F.Cu") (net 2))
 (segment (start 167.4 92.9) (end 164.82 90.32) (width 0.8) (layer "F.Cu") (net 2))
 (segment (start 164.82 90.32) (end 160 90.32) (width 0.8) (layer "F.Cu") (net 2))
 (segment (start 166.202081 110.5) (end 167.4 109.302081) (width 0.8) (layer "F.Cu") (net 2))
 (segment (start 167.4 109.302081) (end 167.4 92.9) (width 0.8) (layer "F.Cu") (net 2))
 (segment (start 123.6 114.276956) (end 131.933044 122.61) (width 0.8) (layer "F.Cu") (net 36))
 (segment (start 121.275 102.128044) (end 123.6 104.453044) (width 0.8) (layer "F.Cu") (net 36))
 (segment (start 121.275 91.74) (end 123.025 89.99) (width 0.8) (layer "F.Cu") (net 36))
 (segment (start 164.112742 92.86) (end 160 92.86) (width 0.8) (layer "F.Cu") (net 36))
 (segment (start 121.275 91.74) (end 121.275 102.128044) (width 0.8) (layer "F.Cu") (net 36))
 (segment (start 161.95 118.784874) (end 161.95 116.791522) (width 0.8) (layer "F.Cu") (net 36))
 (segment (start 162.5 116.241522) (end 162.5 105.2) (width 0.8) (layer "F.Cu") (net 36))
 (segment (start 166.1 101.6) (end 166.1 94.847258) (width 0.8) (layer "F.Cu") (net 36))
 (segment (start 158.124874 122.61) (end 161.95 118.784874) (width 0.8) (layer "F.Cu") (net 36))
 (segment (start 131.933044 122.61) (end 158.124874 122.61) (width 0.8) (layer "F.Cu") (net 36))
 (segment (start 123.6 104.453044) (end 123.6 114.276956) (width 0.8) (layer "F.Cu") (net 36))
 (segment (start 161.95 116.791522) (end 162.5 116.241522) (width 0.8) (layer "F.Cu") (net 36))
 (segment (start 162.5 105.2) (end 166.1 101.6) (width 0.8) (layer "F.Cu") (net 36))
 (segment (start 166.1 94.847258) (end 164.112742 92.86) (width 0.8) (layer "F.Cu") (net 36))
 (segment (start 131.42 73.08) (end 133.25 71.25) (width 0.8) (layer "F.Cu") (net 7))
 (segment (start 131.42 73.08) (end 131.42 84.5) (width 0.8) (layer "F.Cu") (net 7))
 (segment (start 133.25 71.25) (end 133.25 70.5) (width 0.8) (layer "F.Cu") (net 7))
 (segment (start 160.11 95.51) (end 160 95.4) (width 0.8) (layer "F.Cu") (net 28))
 (segment (start 164.5 95.51) (end 160.11 95.51) (width 0.8) (layer "F.Cu") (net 28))
 (segment (start 164.39 100.48) (end 164.5 100.59) (width 0.8) (layer "F.Cu") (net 29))
 (segment (start 160 100.48) (end 164.39 100.48) (width 0.8) (layer "F.Cu") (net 29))
 (segment (start 140.6 108.1) (end 139.83 107.33) (width 0.8) (layer "F.Cu") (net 23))
 (segment (start 142 108.1) (end 140.6 108.1) (width 0.8) (layer "F.Cu") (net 23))
 (segment (start 139.83 107.33) (end 137.5 107.33) (width 0.8) (layer "F.Cu") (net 23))
 (segment (start 137.5 97.17) (end 137.5 99.71) (width 0.8) (layer "F.Cu") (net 46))
 (segment (start 129.88 92.09) (end 128.62 92.09) (width 0.8) (layer "F.Cu") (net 10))
 (segment (start 127.78 91.25) (end 127.78 69.381522) (width 0.8) (layer "F.Cu") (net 10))
 (segment (start 143.202081 72.54) (end 142 72.54) (width 0.8) (layer "F.Cu") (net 10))
 (segment (start 130.161522 67) (end 142.5 67) (width 0.8) (layer "F.Cu") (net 10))
 (segment (start 142.5 67) (end 144 68.5) (width 0.8) (layer "F.Cu") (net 10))
 (segment (start 144 71.742081) (end 143.202081 72.54) (width 0.8) (layer "F.Cu") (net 10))
 (segment (start 127.78 69.381522) (end 130.161522 67) (width 0.8) (layer "F.Cu") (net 10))
 (segment (start 144 68.5) (end 144 71.742081) (width 0.8) (layer "F.Cu") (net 10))
 (segment (start 128.62 92.09) (end 127.78 91.25) (width 0.8) (layer "F.Cu") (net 10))
 (segment (start 138.5 119.073352) (end 140.736648 121.31) (width 0.8) (layer "F.Cu") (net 44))
 (segment (start 140.736648 121.31) (end 154.69 121.31) (width 0.8) (layer "F.Cu") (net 44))
 (segment (start 127.5 111.5) (end 131.2 115.2) (width 0.8) (layer "F.Cu") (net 44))
 (segment (start 154.69 121.31) (end 157.74 118.26) (width 0.8) (layer "F.Cu") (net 44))
 (segment (start 157.74 118.26) (end 160 118.26) (width 0.8) (layer "F.Cu") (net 44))
 (segment (start 129.88 104.79) (end 129.48 104.79) (width 0.8) (layer "F.Cu") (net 44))
 (segment (start 138.5 117.338478) (end 138.5 119.073352) (width 0.8) (layer "F.Cu") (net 44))
 (segment (start 136.361522 115.2) (end 138.5 117.338478) (width 0.8) (layer "F.Cu") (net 44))
 (segment (start 127.5 106.77) (end 127.5 111.5) (width 0.8) (layer "F.Cu") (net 44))
 (segment (start 129.48 104.79) (end 127.5 106.77) (width 0.8) (layer "F.Cu") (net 44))
 (segment (start 131.2 115.2) (end 136.361522 115.2) (width 0.8) (layer "F.Cu") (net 44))
 (segment (start 139.59 92.09) (end 137.5 92.09) (width 0.8) (layer "F.Cu") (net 17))
 (segment (start 140.36 92.86) (end 142 92.86) (width 0.8) (layer "F.Cu") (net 17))
 (segment (start 139.59 92.09) (end 140.36 92.86) (width 0.8) (layer "F.Cu") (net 17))
 (segment (start 139.79 104.79) (end 137.5 104.79) (width 0.8) (layer "F.Cu") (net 22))
 (segment (start 142 105.56) (end 140.56 105.56) (width 0.8) (layer "F.Cu") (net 22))
 (segment (start 140.56 105.56) (end 139.79 104.79) (width 0.8) (layer "F.Cu") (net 22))
 (segment (start 129.88 89.55) (end 129.5675 89.2375) (width 0.8) (layer "F.Cu") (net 9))
 (segment (start 140.6 68.6) (end 142 70) (width 0.8) (layer "F.Cu") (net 9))
 (segment (start 129.5675 69.4325) (end 130.4 68.6) (width 0.8) (layer "F.Cu") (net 9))
 (segment (start 130.4 68.6) (end 140.6 68.6) (width 0.8) (layer "F.Cu") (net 9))
 (segment (start 129.5675 89.2375) (end 129.5675 69.4325) (width 0.8) (layer "F.Cu") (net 9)))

